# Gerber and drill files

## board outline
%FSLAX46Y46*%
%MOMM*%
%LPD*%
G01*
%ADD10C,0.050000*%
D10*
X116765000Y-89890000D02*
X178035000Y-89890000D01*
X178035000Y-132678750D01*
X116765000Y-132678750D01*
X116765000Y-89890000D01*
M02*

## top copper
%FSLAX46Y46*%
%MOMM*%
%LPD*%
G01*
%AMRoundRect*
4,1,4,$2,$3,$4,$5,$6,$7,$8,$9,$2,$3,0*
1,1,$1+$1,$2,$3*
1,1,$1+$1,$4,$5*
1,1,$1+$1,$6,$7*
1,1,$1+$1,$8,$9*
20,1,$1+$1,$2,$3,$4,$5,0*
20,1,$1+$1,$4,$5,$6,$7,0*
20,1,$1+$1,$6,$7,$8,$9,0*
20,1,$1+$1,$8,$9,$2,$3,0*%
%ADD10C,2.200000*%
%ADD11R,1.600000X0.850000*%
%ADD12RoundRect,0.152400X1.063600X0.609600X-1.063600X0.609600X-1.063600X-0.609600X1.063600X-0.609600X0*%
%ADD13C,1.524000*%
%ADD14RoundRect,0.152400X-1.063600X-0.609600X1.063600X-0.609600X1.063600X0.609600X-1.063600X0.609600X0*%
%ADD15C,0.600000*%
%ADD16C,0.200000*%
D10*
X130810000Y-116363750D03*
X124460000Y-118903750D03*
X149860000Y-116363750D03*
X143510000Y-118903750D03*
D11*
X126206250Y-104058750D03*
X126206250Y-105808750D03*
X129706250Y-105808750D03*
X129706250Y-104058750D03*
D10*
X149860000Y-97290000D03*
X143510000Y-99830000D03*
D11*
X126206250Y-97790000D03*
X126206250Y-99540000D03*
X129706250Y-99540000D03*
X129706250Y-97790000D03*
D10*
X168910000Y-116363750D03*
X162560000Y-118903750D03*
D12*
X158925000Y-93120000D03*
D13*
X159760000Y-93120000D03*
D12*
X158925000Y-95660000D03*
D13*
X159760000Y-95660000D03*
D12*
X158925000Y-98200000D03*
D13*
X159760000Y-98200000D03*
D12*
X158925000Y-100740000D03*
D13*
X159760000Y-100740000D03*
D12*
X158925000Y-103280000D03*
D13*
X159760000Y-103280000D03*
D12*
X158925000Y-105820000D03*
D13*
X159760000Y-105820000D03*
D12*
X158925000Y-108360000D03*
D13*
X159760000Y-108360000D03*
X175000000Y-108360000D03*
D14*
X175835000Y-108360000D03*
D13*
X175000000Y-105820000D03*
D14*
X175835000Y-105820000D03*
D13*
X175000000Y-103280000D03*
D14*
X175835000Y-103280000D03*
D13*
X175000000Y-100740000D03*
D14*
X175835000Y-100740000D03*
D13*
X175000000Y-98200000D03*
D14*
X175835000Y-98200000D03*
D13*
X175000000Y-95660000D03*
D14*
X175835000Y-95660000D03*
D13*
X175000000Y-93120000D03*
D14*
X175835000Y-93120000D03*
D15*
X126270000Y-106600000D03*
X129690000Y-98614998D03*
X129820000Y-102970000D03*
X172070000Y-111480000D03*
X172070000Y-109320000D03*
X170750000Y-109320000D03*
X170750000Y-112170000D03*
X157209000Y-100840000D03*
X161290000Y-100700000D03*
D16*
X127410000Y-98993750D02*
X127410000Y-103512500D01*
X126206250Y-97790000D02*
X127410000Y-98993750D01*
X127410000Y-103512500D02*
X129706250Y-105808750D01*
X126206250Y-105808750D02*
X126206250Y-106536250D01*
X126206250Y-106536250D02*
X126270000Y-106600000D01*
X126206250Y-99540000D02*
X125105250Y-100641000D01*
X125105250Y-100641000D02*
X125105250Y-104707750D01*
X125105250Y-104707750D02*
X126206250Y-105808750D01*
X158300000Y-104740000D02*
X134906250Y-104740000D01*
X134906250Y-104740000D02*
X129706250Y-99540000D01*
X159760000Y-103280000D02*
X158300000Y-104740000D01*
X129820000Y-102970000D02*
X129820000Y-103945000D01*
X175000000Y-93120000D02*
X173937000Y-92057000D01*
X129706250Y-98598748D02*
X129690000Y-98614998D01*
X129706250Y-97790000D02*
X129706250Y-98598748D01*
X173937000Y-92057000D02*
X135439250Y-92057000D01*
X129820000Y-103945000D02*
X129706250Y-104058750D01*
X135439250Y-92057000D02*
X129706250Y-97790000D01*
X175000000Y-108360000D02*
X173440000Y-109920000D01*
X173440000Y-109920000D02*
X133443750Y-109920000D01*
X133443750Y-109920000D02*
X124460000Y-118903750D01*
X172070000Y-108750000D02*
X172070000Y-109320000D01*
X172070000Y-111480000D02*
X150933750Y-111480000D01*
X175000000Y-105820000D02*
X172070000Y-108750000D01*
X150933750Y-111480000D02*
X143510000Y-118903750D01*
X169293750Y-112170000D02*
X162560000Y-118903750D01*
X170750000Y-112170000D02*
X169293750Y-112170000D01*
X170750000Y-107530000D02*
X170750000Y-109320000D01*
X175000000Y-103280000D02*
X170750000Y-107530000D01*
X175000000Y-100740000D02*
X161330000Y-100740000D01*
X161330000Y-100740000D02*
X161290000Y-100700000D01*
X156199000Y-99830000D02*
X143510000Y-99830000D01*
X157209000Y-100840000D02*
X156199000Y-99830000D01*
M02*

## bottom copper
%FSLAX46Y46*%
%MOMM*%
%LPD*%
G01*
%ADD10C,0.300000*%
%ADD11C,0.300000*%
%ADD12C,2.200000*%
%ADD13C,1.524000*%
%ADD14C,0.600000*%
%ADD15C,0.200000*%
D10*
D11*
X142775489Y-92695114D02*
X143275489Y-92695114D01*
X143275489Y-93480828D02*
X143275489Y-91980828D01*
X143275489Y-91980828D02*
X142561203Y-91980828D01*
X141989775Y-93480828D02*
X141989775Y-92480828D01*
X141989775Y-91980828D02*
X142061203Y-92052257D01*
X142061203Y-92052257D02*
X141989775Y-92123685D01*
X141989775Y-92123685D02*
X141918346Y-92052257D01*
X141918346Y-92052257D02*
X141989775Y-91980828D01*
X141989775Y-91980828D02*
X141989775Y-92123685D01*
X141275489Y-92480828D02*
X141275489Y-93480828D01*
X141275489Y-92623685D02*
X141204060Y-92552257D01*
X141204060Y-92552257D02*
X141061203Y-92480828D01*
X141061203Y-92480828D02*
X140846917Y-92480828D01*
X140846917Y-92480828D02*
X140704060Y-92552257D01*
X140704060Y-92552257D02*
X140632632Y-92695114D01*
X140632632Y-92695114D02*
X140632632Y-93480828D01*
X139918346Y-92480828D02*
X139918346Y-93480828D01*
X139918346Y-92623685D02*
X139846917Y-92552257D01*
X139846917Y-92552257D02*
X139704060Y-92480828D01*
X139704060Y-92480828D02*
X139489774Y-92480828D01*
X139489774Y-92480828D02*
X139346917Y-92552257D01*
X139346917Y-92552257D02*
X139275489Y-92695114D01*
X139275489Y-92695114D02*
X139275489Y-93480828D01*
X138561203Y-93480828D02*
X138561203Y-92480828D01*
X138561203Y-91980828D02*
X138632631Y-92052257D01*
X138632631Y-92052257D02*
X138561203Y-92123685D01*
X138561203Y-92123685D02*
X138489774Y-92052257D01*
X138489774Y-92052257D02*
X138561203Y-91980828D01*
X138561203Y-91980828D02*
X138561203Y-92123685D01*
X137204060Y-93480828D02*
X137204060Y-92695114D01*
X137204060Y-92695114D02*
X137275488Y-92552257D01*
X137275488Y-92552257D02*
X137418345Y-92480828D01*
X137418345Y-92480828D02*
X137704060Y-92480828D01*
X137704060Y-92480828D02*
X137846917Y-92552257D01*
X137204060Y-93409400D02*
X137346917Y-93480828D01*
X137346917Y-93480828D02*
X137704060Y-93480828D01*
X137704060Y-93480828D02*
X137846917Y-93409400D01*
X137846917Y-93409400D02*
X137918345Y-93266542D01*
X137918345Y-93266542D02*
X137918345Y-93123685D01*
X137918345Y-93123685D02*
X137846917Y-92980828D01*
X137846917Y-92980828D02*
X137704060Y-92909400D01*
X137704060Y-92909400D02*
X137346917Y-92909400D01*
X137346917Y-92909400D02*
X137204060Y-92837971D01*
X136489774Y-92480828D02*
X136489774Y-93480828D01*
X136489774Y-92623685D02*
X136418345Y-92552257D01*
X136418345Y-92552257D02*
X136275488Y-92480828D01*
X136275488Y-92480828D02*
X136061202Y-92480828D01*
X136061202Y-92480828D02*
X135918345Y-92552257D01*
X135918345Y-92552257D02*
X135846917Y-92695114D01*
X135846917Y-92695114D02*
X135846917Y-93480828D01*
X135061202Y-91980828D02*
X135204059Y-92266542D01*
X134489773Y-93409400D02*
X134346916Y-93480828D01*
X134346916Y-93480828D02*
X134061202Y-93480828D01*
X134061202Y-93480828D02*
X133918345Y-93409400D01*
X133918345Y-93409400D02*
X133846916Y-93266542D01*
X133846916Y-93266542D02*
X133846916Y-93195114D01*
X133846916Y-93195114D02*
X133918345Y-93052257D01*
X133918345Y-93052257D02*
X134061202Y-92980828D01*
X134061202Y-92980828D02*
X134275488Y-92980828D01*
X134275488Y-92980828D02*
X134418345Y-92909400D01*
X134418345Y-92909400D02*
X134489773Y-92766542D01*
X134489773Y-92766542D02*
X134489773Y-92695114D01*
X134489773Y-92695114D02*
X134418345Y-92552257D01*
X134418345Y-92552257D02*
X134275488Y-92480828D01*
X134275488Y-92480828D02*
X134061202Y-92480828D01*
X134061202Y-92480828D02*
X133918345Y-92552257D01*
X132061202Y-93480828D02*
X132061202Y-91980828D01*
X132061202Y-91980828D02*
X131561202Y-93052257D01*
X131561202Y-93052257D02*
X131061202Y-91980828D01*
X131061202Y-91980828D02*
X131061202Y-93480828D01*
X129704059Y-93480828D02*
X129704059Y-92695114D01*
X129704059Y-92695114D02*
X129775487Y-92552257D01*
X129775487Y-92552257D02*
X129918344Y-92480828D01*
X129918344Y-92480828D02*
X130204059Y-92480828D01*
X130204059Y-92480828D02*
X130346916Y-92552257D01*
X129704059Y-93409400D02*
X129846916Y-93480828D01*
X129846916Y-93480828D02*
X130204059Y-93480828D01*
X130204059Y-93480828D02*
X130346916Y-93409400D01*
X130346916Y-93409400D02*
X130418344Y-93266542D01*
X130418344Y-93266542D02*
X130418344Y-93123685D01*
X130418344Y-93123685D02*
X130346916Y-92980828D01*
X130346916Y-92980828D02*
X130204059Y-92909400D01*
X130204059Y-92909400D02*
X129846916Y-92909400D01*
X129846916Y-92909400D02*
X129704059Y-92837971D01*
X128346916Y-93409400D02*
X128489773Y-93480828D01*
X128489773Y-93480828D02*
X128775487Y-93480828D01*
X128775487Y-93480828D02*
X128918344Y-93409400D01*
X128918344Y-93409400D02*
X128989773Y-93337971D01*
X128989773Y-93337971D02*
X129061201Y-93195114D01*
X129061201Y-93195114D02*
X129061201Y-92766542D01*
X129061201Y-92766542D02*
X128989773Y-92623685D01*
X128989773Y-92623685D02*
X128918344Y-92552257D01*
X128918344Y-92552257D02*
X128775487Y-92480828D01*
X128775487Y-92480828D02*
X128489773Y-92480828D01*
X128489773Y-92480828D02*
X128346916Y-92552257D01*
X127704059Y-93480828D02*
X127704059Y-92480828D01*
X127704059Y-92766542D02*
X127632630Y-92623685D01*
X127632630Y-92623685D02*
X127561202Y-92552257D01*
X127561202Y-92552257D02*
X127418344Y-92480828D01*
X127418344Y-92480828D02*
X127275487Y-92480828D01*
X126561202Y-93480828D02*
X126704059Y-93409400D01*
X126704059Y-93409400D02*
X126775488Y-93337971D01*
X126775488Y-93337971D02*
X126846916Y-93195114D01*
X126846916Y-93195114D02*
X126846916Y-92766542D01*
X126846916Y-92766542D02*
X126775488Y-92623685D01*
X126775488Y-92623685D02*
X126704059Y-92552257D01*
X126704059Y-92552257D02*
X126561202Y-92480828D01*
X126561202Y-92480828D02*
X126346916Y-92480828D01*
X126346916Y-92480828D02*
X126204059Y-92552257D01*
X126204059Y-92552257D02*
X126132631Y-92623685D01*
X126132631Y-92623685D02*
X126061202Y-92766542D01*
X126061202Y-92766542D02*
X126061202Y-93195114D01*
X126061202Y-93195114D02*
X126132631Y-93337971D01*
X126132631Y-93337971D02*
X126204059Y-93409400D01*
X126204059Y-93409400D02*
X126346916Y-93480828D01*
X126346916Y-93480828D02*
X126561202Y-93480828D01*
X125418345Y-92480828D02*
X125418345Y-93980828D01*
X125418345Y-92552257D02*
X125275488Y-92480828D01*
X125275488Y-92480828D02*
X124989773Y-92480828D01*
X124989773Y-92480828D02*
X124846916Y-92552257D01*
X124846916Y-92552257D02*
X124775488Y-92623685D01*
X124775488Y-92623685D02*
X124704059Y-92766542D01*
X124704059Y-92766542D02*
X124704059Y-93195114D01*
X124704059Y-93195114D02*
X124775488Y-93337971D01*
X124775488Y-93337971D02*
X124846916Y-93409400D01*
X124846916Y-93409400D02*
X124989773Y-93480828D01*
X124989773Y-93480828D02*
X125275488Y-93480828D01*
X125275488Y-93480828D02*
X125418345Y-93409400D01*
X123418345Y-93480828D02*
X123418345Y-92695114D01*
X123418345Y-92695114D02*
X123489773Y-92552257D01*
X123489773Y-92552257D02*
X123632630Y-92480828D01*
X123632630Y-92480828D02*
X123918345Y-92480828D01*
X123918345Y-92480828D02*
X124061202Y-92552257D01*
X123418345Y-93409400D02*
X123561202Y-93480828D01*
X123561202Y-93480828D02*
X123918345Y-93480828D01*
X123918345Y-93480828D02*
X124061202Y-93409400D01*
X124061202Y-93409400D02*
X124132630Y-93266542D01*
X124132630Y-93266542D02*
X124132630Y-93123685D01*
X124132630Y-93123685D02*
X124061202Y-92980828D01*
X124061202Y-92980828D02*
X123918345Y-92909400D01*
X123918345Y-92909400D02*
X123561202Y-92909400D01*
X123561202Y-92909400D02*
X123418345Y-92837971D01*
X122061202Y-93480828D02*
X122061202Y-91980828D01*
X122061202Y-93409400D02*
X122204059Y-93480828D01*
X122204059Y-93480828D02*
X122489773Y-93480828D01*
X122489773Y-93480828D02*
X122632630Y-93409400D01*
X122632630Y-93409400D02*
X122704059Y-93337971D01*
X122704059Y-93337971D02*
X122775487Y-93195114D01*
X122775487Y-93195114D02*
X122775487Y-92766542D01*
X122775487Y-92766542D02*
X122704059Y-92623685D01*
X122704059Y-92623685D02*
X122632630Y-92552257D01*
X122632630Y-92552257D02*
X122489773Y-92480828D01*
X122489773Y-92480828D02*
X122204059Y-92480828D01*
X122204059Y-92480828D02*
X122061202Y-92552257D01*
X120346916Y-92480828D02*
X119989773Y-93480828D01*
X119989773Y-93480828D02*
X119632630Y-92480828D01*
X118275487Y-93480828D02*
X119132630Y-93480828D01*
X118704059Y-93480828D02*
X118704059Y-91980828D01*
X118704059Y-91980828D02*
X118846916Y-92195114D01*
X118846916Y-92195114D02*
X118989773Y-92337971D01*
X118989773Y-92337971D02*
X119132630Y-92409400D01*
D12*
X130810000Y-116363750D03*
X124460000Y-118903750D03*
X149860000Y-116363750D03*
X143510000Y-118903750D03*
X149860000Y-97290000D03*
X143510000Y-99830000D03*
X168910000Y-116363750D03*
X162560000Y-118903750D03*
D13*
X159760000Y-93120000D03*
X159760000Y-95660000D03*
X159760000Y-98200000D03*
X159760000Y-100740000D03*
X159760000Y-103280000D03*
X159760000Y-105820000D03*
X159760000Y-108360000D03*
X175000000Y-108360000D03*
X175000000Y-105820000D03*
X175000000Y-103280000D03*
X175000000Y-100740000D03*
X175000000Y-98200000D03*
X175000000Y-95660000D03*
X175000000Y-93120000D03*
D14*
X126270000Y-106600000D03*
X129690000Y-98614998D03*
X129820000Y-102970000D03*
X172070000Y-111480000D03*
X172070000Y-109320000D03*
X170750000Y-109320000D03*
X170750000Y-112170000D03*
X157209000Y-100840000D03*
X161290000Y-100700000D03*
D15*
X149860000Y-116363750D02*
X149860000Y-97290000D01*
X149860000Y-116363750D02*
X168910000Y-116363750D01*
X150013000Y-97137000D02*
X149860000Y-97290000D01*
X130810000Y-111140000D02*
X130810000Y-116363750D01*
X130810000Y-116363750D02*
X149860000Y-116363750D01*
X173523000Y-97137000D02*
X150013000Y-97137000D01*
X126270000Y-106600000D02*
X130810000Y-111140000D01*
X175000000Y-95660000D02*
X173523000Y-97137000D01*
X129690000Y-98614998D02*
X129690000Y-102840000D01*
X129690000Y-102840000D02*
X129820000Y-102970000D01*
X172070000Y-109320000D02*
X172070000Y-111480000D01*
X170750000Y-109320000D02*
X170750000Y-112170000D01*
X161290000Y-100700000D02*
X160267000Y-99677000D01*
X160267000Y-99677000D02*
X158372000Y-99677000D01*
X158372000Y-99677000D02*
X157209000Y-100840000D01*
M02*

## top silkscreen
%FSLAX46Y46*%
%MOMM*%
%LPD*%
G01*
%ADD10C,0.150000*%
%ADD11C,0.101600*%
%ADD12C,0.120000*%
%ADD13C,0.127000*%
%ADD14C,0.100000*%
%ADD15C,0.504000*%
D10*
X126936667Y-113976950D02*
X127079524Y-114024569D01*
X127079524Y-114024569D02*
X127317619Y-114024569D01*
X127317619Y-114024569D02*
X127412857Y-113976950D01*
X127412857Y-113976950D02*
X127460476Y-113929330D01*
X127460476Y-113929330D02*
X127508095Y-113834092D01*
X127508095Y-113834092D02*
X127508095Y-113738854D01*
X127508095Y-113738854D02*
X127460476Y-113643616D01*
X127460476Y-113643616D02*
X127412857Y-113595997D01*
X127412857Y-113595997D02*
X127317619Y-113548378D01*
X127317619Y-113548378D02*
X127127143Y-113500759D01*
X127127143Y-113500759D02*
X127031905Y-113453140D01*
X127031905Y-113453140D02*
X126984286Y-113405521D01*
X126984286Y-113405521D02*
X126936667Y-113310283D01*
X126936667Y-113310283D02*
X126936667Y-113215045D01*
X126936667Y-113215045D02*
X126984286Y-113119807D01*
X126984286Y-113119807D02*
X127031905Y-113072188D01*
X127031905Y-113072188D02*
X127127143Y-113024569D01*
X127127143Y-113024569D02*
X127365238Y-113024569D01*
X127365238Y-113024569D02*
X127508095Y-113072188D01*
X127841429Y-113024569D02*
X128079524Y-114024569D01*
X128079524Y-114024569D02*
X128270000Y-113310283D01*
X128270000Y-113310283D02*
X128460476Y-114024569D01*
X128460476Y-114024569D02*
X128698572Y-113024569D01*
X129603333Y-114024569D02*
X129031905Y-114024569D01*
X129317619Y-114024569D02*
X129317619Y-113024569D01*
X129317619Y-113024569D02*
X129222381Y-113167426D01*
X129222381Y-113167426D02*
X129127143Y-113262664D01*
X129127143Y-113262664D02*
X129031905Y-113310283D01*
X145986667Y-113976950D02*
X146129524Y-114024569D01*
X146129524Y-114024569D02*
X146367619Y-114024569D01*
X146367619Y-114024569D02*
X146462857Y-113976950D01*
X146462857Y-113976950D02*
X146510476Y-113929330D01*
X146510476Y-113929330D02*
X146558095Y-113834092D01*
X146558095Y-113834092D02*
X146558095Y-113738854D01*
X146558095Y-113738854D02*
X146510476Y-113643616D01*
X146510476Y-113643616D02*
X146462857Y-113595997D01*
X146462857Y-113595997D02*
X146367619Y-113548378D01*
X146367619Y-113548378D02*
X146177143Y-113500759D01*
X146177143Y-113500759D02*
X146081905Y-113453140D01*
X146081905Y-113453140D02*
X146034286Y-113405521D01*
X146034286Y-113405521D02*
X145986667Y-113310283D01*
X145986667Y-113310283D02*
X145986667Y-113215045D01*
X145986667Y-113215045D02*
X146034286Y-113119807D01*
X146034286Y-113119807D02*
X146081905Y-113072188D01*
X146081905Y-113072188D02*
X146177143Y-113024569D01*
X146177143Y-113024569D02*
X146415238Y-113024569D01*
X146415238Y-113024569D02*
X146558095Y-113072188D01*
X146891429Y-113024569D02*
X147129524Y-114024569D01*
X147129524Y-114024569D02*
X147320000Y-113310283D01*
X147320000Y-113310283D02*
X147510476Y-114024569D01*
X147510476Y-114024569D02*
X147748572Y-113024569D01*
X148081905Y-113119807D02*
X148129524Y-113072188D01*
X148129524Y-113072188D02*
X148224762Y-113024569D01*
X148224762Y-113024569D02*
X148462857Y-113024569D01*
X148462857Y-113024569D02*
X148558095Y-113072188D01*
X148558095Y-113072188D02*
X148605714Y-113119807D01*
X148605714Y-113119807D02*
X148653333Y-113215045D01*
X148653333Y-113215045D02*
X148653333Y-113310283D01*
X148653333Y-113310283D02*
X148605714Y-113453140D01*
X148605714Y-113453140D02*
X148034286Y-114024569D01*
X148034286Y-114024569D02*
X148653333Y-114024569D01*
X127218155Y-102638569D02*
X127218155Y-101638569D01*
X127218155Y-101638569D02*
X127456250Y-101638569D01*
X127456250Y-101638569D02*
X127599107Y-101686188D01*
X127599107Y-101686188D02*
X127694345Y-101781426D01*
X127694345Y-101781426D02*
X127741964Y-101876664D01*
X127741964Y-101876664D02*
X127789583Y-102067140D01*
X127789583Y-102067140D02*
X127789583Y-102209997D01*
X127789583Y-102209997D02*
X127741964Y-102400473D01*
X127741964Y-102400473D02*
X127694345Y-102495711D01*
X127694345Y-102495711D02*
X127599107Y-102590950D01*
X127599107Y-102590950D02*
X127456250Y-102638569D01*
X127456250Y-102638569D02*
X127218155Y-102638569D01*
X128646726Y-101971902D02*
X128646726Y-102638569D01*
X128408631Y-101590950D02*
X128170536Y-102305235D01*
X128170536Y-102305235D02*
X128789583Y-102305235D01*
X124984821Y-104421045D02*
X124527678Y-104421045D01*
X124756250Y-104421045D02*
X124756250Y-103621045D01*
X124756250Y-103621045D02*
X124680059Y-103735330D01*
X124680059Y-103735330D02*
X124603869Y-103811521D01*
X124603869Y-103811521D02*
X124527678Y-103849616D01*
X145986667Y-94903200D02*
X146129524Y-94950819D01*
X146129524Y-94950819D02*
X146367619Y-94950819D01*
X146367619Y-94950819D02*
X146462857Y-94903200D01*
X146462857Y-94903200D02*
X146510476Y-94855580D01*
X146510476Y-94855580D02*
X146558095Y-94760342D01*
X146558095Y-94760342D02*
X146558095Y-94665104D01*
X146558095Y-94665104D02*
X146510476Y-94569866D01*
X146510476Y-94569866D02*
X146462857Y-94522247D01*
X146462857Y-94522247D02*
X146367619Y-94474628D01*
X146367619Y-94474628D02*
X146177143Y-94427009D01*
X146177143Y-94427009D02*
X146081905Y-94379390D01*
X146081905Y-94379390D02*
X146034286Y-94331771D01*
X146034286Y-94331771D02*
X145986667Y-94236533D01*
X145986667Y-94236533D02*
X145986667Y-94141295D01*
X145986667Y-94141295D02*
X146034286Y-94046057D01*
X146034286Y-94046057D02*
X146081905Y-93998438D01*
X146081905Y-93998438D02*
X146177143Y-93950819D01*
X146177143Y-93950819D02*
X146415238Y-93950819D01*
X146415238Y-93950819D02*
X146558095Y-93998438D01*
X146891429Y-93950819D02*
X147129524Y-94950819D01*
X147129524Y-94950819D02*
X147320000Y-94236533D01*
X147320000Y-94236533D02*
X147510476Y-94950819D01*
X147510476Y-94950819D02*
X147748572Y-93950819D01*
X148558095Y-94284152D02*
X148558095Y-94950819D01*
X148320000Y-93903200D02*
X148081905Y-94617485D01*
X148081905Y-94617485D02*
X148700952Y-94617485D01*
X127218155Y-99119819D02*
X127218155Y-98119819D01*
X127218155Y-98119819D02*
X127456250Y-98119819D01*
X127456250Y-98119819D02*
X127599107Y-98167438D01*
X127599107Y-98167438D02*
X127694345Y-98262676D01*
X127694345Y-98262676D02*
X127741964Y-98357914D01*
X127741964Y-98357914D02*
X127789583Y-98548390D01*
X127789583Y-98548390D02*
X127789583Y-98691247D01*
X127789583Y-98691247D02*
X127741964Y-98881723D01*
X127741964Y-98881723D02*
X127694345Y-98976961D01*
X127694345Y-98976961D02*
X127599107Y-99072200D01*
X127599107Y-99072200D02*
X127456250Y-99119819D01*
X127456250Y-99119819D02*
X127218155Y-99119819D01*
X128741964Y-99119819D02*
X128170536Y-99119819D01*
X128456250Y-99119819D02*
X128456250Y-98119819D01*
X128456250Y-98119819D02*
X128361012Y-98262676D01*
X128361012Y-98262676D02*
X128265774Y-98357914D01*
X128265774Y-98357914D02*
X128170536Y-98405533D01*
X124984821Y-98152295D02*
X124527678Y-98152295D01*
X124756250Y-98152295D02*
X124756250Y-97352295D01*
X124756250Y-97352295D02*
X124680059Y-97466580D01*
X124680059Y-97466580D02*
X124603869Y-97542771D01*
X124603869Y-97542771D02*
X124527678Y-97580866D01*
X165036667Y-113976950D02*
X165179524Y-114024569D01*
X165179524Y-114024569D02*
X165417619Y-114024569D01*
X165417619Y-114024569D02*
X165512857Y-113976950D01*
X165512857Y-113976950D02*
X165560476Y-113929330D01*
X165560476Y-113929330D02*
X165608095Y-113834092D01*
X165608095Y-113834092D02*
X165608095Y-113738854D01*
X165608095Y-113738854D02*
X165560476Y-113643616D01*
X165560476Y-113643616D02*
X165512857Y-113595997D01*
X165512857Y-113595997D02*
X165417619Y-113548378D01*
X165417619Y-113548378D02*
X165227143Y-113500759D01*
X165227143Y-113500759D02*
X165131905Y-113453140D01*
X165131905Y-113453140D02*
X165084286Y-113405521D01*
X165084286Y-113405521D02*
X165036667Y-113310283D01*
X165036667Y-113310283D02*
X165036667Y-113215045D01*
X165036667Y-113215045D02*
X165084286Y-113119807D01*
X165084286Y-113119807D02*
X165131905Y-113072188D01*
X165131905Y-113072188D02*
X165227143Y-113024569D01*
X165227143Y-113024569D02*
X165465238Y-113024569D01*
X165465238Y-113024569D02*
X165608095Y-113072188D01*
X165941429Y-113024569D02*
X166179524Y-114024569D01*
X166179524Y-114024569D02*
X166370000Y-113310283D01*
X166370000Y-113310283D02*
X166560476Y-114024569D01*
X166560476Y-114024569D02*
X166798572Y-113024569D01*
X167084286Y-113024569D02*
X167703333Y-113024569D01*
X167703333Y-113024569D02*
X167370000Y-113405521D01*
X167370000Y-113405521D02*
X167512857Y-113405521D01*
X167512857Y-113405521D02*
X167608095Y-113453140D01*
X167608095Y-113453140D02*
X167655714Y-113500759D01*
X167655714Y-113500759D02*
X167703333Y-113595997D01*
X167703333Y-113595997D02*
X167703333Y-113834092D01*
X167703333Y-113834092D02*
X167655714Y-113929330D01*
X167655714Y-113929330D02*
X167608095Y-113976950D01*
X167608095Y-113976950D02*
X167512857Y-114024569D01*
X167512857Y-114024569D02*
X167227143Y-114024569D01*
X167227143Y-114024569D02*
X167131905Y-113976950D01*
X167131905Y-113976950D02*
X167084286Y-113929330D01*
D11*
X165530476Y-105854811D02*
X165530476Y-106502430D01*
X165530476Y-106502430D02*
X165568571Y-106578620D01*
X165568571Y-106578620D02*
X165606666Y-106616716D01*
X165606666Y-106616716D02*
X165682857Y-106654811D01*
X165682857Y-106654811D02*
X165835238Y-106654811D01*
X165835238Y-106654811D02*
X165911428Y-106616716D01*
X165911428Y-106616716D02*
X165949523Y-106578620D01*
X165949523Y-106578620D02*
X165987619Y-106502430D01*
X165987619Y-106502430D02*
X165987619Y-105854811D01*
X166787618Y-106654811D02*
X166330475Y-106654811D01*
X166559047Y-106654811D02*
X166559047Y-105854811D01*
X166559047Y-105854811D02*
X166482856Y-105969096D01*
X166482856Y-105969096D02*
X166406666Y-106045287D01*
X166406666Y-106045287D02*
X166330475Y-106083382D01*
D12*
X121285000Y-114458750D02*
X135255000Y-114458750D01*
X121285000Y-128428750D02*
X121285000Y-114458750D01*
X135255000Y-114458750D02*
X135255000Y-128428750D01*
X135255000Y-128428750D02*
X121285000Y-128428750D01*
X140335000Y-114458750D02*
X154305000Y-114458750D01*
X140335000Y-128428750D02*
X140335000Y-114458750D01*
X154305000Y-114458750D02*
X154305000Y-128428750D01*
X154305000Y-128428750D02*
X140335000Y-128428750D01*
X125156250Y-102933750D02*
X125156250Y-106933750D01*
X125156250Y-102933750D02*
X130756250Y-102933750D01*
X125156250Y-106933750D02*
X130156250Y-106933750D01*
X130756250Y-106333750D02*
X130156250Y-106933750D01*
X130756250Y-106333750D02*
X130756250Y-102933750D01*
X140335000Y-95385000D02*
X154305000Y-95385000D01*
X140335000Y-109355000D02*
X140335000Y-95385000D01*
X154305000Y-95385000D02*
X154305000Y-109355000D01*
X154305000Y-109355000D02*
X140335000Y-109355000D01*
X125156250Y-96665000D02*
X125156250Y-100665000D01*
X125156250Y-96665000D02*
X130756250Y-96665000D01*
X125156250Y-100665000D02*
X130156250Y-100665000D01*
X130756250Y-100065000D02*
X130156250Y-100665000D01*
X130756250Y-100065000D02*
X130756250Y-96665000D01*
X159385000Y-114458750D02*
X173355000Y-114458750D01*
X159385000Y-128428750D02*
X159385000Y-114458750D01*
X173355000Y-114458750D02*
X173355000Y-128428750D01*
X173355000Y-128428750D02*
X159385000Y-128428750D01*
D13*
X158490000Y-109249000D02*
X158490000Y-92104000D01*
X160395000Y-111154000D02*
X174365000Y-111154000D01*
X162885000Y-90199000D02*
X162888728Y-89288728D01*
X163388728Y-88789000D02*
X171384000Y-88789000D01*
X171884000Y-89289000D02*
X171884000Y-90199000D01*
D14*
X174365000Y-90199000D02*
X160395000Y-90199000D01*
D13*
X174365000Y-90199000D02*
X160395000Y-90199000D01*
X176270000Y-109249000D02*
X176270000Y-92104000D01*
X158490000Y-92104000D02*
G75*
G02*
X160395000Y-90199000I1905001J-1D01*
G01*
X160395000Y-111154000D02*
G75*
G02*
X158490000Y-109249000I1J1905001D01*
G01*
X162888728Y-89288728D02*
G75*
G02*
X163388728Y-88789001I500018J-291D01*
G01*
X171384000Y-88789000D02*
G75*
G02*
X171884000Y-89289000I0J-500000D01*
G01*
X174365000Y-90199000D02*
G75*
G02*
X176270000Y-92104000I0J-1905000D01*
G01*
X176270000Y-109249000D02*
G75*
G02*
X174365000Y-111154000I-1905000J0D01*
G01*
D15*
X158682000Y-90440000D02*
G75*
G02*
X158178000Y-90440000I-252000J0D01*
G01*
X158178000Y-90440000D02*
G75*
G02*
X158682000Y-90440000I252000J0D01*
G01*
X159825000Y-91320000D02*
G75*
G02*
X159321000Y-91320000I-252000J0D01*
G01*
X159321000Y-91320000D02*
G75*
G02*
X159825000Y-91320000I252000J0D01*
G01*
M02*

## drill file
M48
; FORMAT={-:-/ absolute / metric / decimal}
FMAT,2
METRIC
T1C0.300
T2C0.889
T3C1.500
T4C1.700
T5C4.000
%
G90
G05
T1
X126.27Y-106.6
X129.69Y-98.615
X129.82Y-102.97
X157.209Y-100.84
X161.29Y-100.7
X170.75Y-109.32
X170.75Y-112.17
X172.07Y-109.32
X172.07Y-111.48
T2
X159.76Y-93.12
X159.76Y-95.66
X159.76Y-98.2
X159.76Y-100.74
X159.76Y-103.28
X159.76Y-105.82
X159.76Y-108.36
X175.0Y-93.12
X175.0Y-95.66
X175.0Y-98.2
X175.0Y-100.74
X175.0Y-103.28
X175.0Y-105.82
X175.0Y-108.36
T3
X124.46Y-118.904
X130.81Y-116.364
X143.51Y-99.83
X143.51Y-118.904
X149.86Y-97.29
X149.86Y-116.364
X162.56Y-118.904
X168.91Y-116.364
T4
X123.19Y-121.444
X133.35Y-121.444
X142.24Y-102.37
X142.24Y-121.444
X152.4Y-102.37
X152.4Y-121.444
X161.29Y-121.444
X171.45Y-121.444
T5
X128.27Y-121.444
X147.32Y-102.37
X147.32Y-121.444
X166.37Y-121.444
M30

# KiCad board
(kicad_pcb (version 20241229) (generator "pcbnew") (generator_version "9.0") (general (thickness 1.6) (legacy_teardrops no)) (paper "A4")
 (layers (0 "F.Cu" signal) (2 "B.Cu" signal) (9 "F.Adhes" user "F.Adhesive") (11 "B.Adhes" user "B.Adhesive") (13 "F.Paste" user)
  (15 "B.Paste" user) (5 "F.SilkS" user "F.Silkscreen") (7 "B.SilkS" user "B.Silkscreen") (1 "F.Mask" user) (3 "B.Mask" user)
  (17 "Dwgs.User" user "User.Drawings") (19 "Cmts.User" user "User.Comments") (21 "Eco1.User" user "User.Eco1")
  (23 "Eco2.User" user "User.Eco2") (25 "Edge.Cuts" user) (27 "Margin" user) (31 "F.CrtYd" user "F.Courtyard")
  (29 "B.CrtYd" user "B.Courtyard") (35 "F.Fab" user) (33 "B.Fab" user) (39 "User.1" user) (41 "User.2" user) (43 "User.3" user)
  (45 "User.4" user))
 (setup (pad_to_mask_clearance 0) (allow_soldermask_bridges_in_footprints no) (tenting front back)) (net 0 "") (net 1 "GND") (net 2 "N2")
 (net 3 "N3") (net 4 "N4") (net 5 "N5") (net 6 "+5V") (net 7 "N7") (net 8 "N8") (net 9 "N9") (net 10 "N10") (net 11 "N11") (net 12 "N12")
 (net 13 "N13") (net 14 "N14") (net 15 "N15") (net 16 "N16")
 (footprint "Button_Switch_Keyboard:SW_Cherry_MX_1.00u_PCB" (layer "F.Cu") (at 130.81 116.36375)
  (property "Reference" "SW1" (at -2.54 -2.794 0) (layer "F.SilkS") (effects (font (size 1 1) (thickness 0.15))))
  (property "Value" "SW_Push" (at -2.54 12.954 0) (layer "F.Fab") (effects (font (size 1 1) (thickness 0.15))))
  (fp_line (start -9.525 -1.905) (end 4.445 -1.905) (stroke (width 0.12) (type solid)) (layer "F.SilkS"))
  (fp_line (start -9.525 12.065) (end -9.525 -1.905) (stroke (width 0.12) (type solid)) (layer "F.SilkS"))
  (fp_line (start 4.445 -1.905) (end 4.445 12.065) (stroke (width 0.12) (type solid)) (layer "F.SilkS"))
  (fp_line (start 4.445 12.065) (end -9.525 12.065) (stroke (width 0.12) (type solid)) (layer "F.SilkS"))
  (pad "" np_thru_hole circle (at -7.62 5.08) (size 1.7 1.7) (drill 1.7) (layers "*.Cu" "*.Mask"))
  (pad "" np_thru_hole circle (at -2.54 5.08) (size 4 4) (drill 4) (layers "*.Cu" "*.Mask"))
  (pad "" np_thru_hole circle (at 2.54 5.08) (size 1.7 1.7) (drill 1.7) (layers "*.Cu" "*.Mask"))
  (pad "1" thru_hole circle (at 0 0) (size 2.2 2.2) (drill 1.5) (layers "*.Cu" "*.Mask") (remove_unused_layers no) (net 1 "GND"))
  (pad "2" thru_hole circle (at -6.35 2.54) (size 2.2 2.2) (drill 1.5) (layers "*.Cu" "*.Mask") (remove_unused_layers no) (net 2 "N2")))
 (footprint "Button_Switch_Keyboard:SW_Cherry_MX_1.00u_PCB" (layer "F.Cu") (at 149.86 116.36375)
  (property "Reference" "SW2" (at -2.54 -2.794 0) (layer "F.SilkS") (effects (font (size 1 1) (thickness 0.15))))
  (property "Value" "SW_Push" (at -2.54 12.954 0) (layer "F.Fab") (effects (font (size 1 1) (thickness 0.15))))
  (fp_line (start -9.525 -1.905) (end 4.445 -1.905) (stroke (width 0.12) (type solid)) (layer "F.SilkS"))
  (fp_line (start -9.525 12.065) (end -9.525 -1.905) (stroke (width 0.12) (type solid)) (layer "F.SilkS"))
  (fp_line (start 4.445 -1.905) (end 4.445 12.065) (stroke (width 0.12) (type solid)) (layer "F.SilkS"))
  (fp_line (start 4.445 12.065) (end -9.525 12.065) (stroke (width 0.12) (type solid)) (layer "F.SilkS"))
  (pad "" np_thru_hole circle (at -7.62 5.08) (size 1.7 1.7) (drill 1.7) (layers "*.Cu" "*.Mask"))
  (pad "" np_thru_hole circle (at -2.54 5.08) (size 4 4) (drill 4) (layers "*.Cu" "*.Mask"))
  (pad "" np_thru_hole circle (at 2.54 5.08) (size 1.7 1.7) (drill 1.7) (layers "*.Cu" "*.Mask"))
  (pad "1" thru_hole circle (at 0 0) (size 2.2 2.2) (drill 1.5) (layers "*.Cu" "*.Mask") (remove_unused_layers no) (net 1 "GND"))
  (pad "2" thru_hole circle (at -6.35 2.54) (size 2.2 2.2) (drill 1.5) (layers "*.Cu" "*.Mask") (remove_unused_layers no) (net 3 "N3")))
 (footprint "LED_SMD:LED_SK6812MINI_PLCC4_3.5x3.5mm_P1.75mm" (layer "F.Cu") (at 127.95625 104.93375)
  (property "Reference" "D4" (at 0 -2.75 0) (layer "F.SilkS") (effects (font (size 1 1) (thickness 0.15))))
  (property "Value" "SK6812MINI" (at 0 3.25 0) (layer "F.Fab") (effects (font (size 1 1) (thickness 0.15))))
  (fp_line (start -2.8 -2) (end -2.8 2) (stroke (width 0.12) (type default)) (layer "F.SilkS"))
  (fp_line (start -2.8 -2) (end 2.8 -2) (stroke (width 0.12) (type solid)) (layer "F.SilkS"))
  (fp_line (start -2.8 2) (end 2.2 2) (stroke (width 0.12) (type solid)) (layer "F.SilkS"))
  (fp_line (start 2.8 1.4) (end 2.2 2) (stroke (width 0.12) (type default)) (layer "F.SilkS"))
  (fp_line (start 2.8 1.4) (end 2.8 -2) (stroke (width 0.12) (type solid)) (layer "F.SilkS"))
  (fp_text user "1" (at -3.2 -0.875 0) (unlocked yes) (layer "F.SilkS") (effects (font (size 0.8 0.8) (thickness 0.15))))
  (pad "1" smd rect (at -1.75 -0.875) (size 1.6 0.85) (layers "F.Cu" "F.Mask" "F.Paste") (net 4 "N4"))
  (pad "2" smd rect (at -1.75 0.875) (size 1.6 0.85) (layers "F.Cu" "F.Mask" "F.Paste") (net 1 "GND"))
  (pad "3" smd rect (at 1.75 0.875) (size 1.6 0.85) (layers "F.Cu" "F.Mask" "F.Paste") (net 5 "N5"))
  (pad "4" smd rect (at 1.75 -0.875) (size 1.6 0.85) (layers "F.Cu" "F.Mask" "F.Paste") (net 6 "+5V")))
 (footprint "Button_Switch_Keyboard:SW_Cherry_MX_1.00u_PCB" (layer "F.Cu") (at 149.86 97.29)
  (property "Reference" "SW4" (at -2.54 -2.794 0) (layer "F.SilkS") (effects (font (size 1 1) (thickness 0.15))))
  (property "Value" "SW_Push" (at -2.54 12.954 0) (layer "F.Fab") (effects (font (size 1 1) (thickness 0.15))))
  (fp_line (start -9.525 -1.905) (end 4.445 -1.905) (stroke (width 0.12) (type solid)) (layer "F.SilkS"))
  (fp_line (start -9.525 12.065) (end -9.525 -1.905) (stroke (width 0.12) (type solid)) (layer "F.SilkS"))
  (fp_line (start 4.445 -1.905) (end 4.445 12.065) (stroke (width 0.12) (type solid)) (layer "F.SilkS"))
  (fp_line (start 4.445 12.065) (end -9.525 12.065) (stroke (width 0.12) (type solid)) (layer "F.SilkS"))
  (pad "" np_thru_hole circle (at -7.62 5.08) (size 1.7 1.7) (drill 1.7) (layers "*.Cu" "*.Mask"))
  (pad "" np_thru_hole circle (at -2.54 5.08) (size 4 4) (drill 4) (layers "*.Cu" "*.Mask"))
  (pad "" np_thru_hole circle (at 2.54 5.08) (size 1.7 1.7) (drill 1.7) (layers "*.Cu" "*.Mask"))
  (pad "1" thru_hole circle (at 0 0) (size 2.2 2.2) (drill 1.5) (layers "*.Cu" "*.Mask") (remove_unused_layers no) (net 1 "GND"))
  (pad "2" thru_hole circle (at -6.35 2.54) (size 2.2 2.2) (drill 1.5) (layers "*.Cu" "*.Mask") (remove_unused_layers no) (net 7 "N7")))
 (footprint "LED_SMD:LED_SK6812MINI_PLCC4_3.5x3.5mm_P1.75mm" (layer "F.Cu") (at 127.95625 98.665)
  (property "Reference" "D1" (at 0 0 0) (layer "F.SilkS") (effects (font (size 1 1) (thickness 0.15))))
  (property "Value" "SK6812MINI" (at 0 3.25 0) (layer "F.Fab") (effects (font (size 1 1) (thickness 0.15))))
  (fp_line (start -2.8 -2) (end -2.8 2) (stroke (width 0.12) (type default)) (layer "F.SilkS"))
  (fp_line (start -2.8 -2) (end 2.8 -2) (stroke (width 0.12) (type solid)) (layer "F.SilkS"))
  (fp_line (start -2.8 2) (end 2.2 2) (stroke (width 0.12) (type solid)) (layer "F.SilkS"))
  (fp_line (start 2.8 1.4) (end 2.2 2) (stroke (width 0.12) (type default)) (layer "F.SilkS"))
  (fp_line (start 2.8 1.4) (end 2.8 -2) (stroke (width 0.12) (type solid)) (layer "F.SilkS"))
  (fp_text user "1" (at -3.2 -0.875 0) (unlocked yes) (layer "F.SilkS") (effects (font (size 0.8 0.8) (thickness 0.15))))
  (pad "1" smd rect (at -1.75 -0.875) (size 1.6 0.85) (layers "F.Cu" "F.Mask" "F.Paste") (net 5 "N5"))
  (pad "2" smd rect (at -1.75 0.875) (size 1.6 0.85) (layers "F.Cu" "F.Mask" "F.Paste") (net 1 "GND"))
  (pad "3" smd rect (at 1.75 0.875) (size 1.6 0.85) (layers "F.Cu" "F.Mask" "F.Paste") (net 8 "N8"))
  (pad "4" smd rect (at 1.75 -0.875) (size 1.6 0.85) (layers "F.Cu" "F.Mask" "F.Paste") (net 6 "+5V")))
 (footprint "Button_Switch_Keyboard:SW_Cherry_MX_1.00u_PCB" (layer "F.Cu") (at 168.91 116.36375)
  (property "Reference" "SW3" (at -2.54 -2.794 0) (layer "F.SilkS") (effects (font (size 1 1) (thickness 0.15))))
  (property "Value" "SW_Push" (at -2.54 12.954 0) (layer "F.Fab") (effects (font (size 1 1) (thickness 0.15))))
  (fp_line (start -9.525 -1.905) (end 4.445 -1.905) (stroke (width 0.12) (type solid)) (layer "F.SilkS"))
  (fp_line (start -9.525 12.065) (end -9.525 -1.905) (stroke (width 0.12) (type solid)) (layer "F.SilkS"))
  (fp_line (start 4.445 -1.905) (end 4.445 12.065) (stroke (width 0.12) (type solid)) (layer "F.SilkS"))
  (fp_line (start 4.445 12.065) (end -9.525 12.065) (stroke (width 0.12) (type solid)) (layer "F.SilkS"))
  (pad "" np_thru_hole circle (at -7.62 5.08) (size 1.7 1.7) (drill 1.7) (layers "*.Cu" "*.Mask"))
  (pad "" np_thru_hole circle (at -2.54 5.08) (size 4 4) (drill 4) (layers "*.Cu" "*.Mask"))
  (pad "" np_thru_hole circle (at 2.54 5.08) (size 1.7 1.7) (drill 1.7) (layers "*.Cu" "*.Mask"))
  (pad "1" thru_hole circle (at 0 0) (size 2.2 2.2) (drill 1.5) (layers "*.Cu" "*.Mask") (remove_unused_layers no) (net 1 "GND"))
  (pad "2" thru_hole circle (at -6.35 2.54) (size 2.2 2.2) (drill 1.5) (layers "*.Cu" "*.Mask") (remove_unused_layers no) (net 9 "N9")))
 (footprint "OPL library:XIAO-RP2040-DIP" (layer "F.Cu") (at 167.38 100.74)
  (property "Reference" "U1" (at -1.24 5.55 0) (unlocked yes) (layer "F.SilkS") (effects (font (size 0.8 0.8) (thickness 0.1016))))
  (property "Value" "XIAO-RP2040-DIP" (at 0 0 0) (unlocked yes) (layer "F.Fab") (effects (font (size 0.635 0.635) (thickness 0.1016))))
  (fp_line (start -8.89 8.509) (end -8.89 -8.636) (stroke (width 0.127) (type solid)) (layer "F.SilkS"))
  (fp_line (start -6.985 10.414) (end 6.985 10.414) (stroke (width 0.127) (type solid)) (layer "F.SilkS"))
  (fp_line (start -4.495 -10.541) (end -4.491272 -11.451272) (stroke (width 0.127) (type solid)) (layer "F.SilkS"))
  (fp_line (start -3.991272 -11.951) (end 4.004 -11.951) (stroke (width 0.127) (type solid)) (layer "F.SilkS"))
  (fp_line (start 4.504 -11.451) (end 4.504 -10.541) (stroke (width 0.127) (type solid)) (layer "F.SilkS"))
  (fp_line (start 6.985 -10.541) (end -6.985 -10.541) (stroke (width 0.1) (type solid)) (layer "F.SilkS"))
  (fp_line (start 6.985 -10.541) (end -6.985 -10.541) (stroke (width 0.127) (type solid)) (layer "F.SilkS"))
  (fp_line (start 8.89 8.509) (end 8.89 -8.636) (stroke (width 0.127) (type solid)) (layer "F.SilkS"))
  (fp_arc (start -8.89 -8.636) (mid -8.332038 -9.983038) (end -6.985 -10.541) (stroke (width 0.127) (type solid)) (layer "F.SilkS"))
  (fp_arc (start -6.985 10.414) (mid -8.332038 9.856038) (end -8.89 8.509) (stroke (width 0.127) (type solid)) (layer "F.SilkS"))
  (fp_arc (start -4.491272 -11.451272) (mid -4.344728 -11.80464) (end -3.991272 -11.951) (stroke (width 0.127) (type default))
   (layer "F.SilkS"))
  (fp_arc (start 4.004 -11.951) (mid 4.357553 -11.804553) (end 4.504 -11.451) (stroke (width 0.127) (type default)) (layer "F.SilkS"))
  (fp_arc (start 6.985 -10.541) (mid 8.332038 -9.983038) (end 8.89 -8.636) (stroke (width 0.127) (type solid)) (layer "F.SilkS"))
  (fp_arc (start 8.89 8.509) (mid 8.332038 9.856038) (end 6.985 10.414) (stroke (width 0.127) (type solid)) (layer "F.SilkS"))
  (fp_circle (center -8.95 -10.3) (end -8.95 -10.554) (stroke (width 0.5) (type solid)) (fill yes) (layer "F.SilkS"))
  (fp_circle (center -7.807 -9.42) (end -7.807 -9.674) (stroke (width 0.5) (type solid)) (fill yes) (layer "F.SilkS"))
  (pad "1" smd roundrect (at -8.455 -7.62 180) (size 2.432 1.524) (layers "F.Cu" "F.Mask") (roundrect_rratio 0.1) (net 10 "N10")
   (thermal_bridge_angle 45))
  (pad "1" thru_hole circle (at -7.62 -7.62 180) (size 1.524 1.524) (drill 0.889) (layers "*.Cu" "*.Mask") (remove_unused_layers no)
   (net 10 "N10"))
  (pad "2" smd roundrect (at -8.455 -5.08 180) (size 2.432 1.524) (layers "F.Cu" "F.Mask") (roundrect_rratio 0.1) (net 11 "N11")
   (thermal_bridge_angle 45))
  (pad "2" thru_hole circle (at -7.62 -5.08 180) (size 1.524 1.524) (drill 0.889) (layers "*.Cu" "*.Mask") (remove_unused_layers no)
   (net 11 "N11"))
  (pad "3" smd roundrect (at -8.455 -2.54 180) (size 2.432 1.524) (layers "F.Cu" "F.Mask") (roundrect_rratio 0.1) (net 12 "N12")
   (thermal_bridge_angle 45))
  (pad "3" thru_hole circle (at -7.62 -2.54 180) (size 1.524 1.524) (drill 0.889) (layers "*.Cu" "*.Mask") (remove_unused_layers no)
   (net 12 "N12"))
  (pad "4" smd roundrect (at -8.455 0 180) (size 2.432 1.524) (layers "F.Cu" "F.Mask") (roundrect_rratio 0.1) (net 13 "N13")
   (thermal_bridge_angle 45))
  (pad "4" thru_hole circle (at -7.62 0 180) (size 1.524 1.524) (drill 0.889) (layers "*.Cu" "*.Mask") (remove_unused_layers no)
   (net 13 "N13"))
  (pad "5" smd roundrect (at -8.455 2.54 180) (size 2.432 1.524) (layers "F.Cu" "F.Mask") (roundrect_rratio 0.1) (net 8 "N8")
   (thermal_bridge_angle 45))
  (pad "5" thru_hole circle (at -7.62 2.54 180) (size 1.524 1.524) (drill 0.889) (layers "*.Cu" "*.Mask") (remove_unused_layers no)
   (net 8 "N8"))
  (pad "6" smd roundrect (at -8.455 5.08 180) (size 2.432 1.524) (layers "F.Cu" "F.Mask") (roundrect_rratio 0.1) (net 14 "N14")
   (thermal_bridge_angle 45))
  (pad "6" thru_hole circle (at -7.62 5.08 180) (size 1.524 1.524) (drill 0.889) (layers "*.Cu" "*.Mask") (remove_unused_layers no)
   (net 14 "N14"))
  (pad "7" smd roundrect (at -8.455 7.62 180) (size 2.432 1.524) (layers "F.Cu" "F.Mask") (roundrect_rratio 0.1) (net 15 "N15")
   (thermal_bridge_angle 45))
  (pad "7" thru_hole circle (at -7.62 7.62 180) (size 1.524 1.524) (drill 0.889) (layers "*.Cu" "*.Mask") (remove_unused_layers no)
   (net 15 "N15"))
  (pad "8" thru_hole circle (at 7.62 7.62) (size 1.524 1.524) (drill 0.889) (layers "*.Cu" "*.Mask") (remove_unused_layers no) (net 2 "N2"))
  (pad "8" smd roundrect (at 8.455 7.62) (size 2.432 1.524) (layers "F.Cu" "F.Mask") (roundrect_rratio 0.1) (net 2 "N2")
   (thermal_bridge_angle 45))
  (pad "9" thru_hole circle (at 7.62 5.08) (size 1.524 1.524) (drill 0.889) (layers "*.Cu" "*.Mask") (remove_unused_layers no) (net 3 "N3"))
  (pad "9" smd roundrect (at 8.455 5.08) (size 2.432 1.524) (layers "F.Cu" "F.Mask") (roundrect_rratio 0.1) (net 3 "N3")
   (thermal_bridge_angle 45))
  (pad "10" thru_hole circle (at 7.62 2.54) (size 1.524 1.524) (drill 0.889) (layers "*.Cu" "*.Mask") (remove_unused_layers no) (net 9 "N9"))
  (pad "10" smd roundrect (at 8.455 2.54) (size 2.432 1.524) (layers "F.Cu" "F.Mask") (roundrect_rratio 0.1) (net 9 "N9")
   (thermal_bridge_angle 45))
  (pad "11" thru_hole circle (at 7.62 0) (size 1.524 1.524) (drill 0.889) (layers "*.Cu" "*.Mask") (remove_unused_layers no) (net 7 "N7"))
  (pad "11" smd roundrect (at 8.455 0) (size 2.432 1.524) (layers "F.Cu" "F.Mask") (roundrect_rratio 0.1) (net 7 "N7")
   (thermal_bridge_angle 45))
  (pad "12" thru_hole circle (at 7.62 -2.54) (size 1.524 1.524) (drill 0.889) (layers "*.Cu" "*.Mask") (remove_unused_layers no)
   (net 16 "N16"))
  (pad "12" smd roundrect (at 8.455 -2.54) (size 2.432 1.524) (layers "F.Cu" "F.Mask") (roundrect_rratio 0.1) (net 16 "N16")
   (thermal_bridge_angle 45))
  (pad "13" thru_hole circle (at 7.62 -5.08) (size 1.524 1.524) (drill 0.889) (layers "*.Cu" "*.Mask") (remove_unused_layers no)
   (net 1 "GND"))
  (pad "13" smd roundrect (at 8.455 -5.08) (size 2.432 1.524) (layers "F.Cu" "F.Mask") (roundrect_rratio 0.1) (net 1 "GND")
   (thermal_bridge_angle 45))
  (pad "14" thru_hole circle (at 7.62 -7.62) (size 1.524 1.524) (drill 0.889) (layers "*.Cu" "*.Mask") (remove_unused_layers no)
   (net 6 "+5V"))
  (pad "14" smd roundrect (at 8.455 -7.62) (size 2.432 1.524) (layers "F.Cu" "F.Mask") (roundrect_rratio 0.1) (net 6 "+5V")
   (thermal_bridge_angle 45)))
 (gr_rect (start 116.765 89.89) (end 178.035 132.67875) (stroke (width 0.05) (type default)) (fill no) (layer "Edge.Cuts"))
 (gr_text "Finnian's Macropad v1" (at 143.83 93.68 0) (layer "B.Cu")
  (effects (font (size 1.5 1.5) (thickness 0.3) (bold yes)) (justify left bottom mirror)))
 (segment (start 127.41 98.99375) (end 127.41 103.5125) (width 0.2) (layer "F.Cu") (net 5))
 (segment (start 126.20625 97.79) (end 127.41 98.99375) (width 0.2) (layer "F.Cu") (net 5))
 (segment (start 127.41 103.5125) (end 129.70625 105.80875) (width 0.2) (layer "F.Cu") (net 5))
 (segment (start 126.20625 105.80875) (end 126.20625 106.53625) (width 0.2) (layer "F.Cu") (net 1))
 (segment (start 126.20625 106.53625) (end 126.27 106.6) (width 0.2) (layer "F.Cu") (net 1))
 (segment (start 126.20625 99.54) (end 125.10525 100.641) (width 0.2) (layer "F.Cu") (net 1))
 (segment (start 125.10525 100.641) (end 125.10525 104.70775) (width 0.2) (layer "F.Cu") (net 1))
 (segment (start 125.10525 104.70775) (end 126.20625 105.80875) (width 0.2) (layer "F.Cu") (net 1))
 (via (at 126.27 106.6) (size 0.6) (drill 0.3) (layers "F.Cu" "B.Cu") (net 1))
 (segment (start 149.86 116.36375) (end 149.86 97.29) (width 0.2) (layer "B.Cu") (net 1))
 (segment (start 149.86 116.36375) (end 168.91 116.36375) (width 0.2) (layer "B.Cu") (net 1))
 (segment (start 150.013 97.137) (end 149.86 97.29) (width 0.2) (layer "B.Cu") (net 1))
 (segment (start 130.81 111.14) (end 130.81 116.36375) (width 0.2) (layer "B.Cu") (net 1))
 (segment (start 130.81 116.36375) (end 149.86 116.36375) (width 0.2) (layer "B.Cu") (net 1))
 (segment (start 173.523 97.137) (end 150.013 97.137) (width 0.2) (layer "B.Cu") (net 1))
 (segment (start 126.27 106.6) (end 130.81 111.14) (width 0.2) (layer "B.Cu") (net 1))
 (segment (start 175 95.66) (end 173.523 97.137) (width 0.2) (layer "B.Cu") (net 1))
 (segment (start 158.3 104.74) (end 134.90625 104.74) (width 0.2) (layer "F.Cu") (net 8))
 (segment (start 134.90625 104.74) (end 129.70625 99.54) (width 0.2) (layer "F.Cu") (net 8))
 (segment (start 159.76 103.28) (end 158.3 104.74) (width 0.2) (layer "F.Cu") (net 8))
 (segment (start 129.82 102.97) (end 129.82 103.945) (width 0.2) (layer "F.Cu") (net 6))
 (segment (start 175 93.12) (end 173.937 92.057) (width 0.2) (layer "F.Cu") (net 6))
 (segment (start 129.70625 98.598748) (end 129.69 98.614998) (width 0.2) (layer "F.Cu") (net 6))
 (segment (start 129.70625 97.79) (end 129.70625 98.598748) (width 0.2) (layer "F.Cu") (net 6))
 (segment (start 173.937 92.057) (end 135.43925 92.057) (width 0.2) (layer "F.Cu") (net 6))
 (segment (start 129.82 103.945) (end 129.70625 104.05875) (width 0.2) (layer "F.Cu") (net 6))
 (segment (start 135.43925 92.057) (end 129.70625 97.79) (width 0.2) (layer "F.Cu") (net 6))
 (via (at 129.69 98.614998) (size 0.6) (drill 0.3) (layers "F.Cu" "B.Cu") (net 6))
 (via (at 129.82 102.97) (size 0.6) (drill 0.3) (layers "F.Cu" "B.Cu") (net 6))
 (segment (start 129.69 98.614998) (end 129.69 102.84) (width 0.2) (layer "B.Cu") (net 6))
 (segment (start 129.69 102.84) (end 129.82 102.97) (width 0.2) (layer "B.Cu") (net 6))
 (segment (start 175 108.36) (end 173.44 109.92) (width 0.2) (layer "F.Cu") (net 2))
 (segment (start 173.44 109.92) (end 133.44375 109.92) (width 0.2) (layer "F.Cu") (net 2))
 (segment (start 133.44375 109.92) (end 124.46 118.90375) (width 0.2) (layer "F.Cu") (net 2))
 (segment (start 172.07 108.75) (end 172.07 109.32) (width 0.2) (layer "F.Cu") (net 3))
 (segment (start 172.07 111.48) (end 150.93375 111.48) (width 0.2) (layer "F.Cu") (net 3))
 (segment (start 175 105.82) (end 172.07 108.75) (width 0.2) (layer "F.Cu") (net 3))
 (segment (start 150.93375 111.48) (end 143.51 118.90375) (width 0.2) (layer "F.Cu") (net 3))
 (via (at 172.07 111.48) (size 0.6) (drill 0.3) (layers "F.Cu" "B.Cu") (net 3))
 (via (at 172.07 109.32) (size 0.6) (drill 0.3) (layers "F.Cu" "B.Cu") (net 3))
 (segment (start 172.07 109.32) (end 172.07 111.48) (width 0.2) (layer "B.Cu") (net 3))
 (segment (start 169.29375 112.17) (end 162.56 118.90375) (width 0.2) (layer "F.Cu") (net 9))
 (segment (start 170.75 112.17) (end 169.29375 112.17) (width 0.2) (layer "F.Cu") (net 9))
 (segment (start 170.75 107.53) (end 170.75 109.32) (width 0.2) (layer "F.Cu") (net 9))
 (segment (start 175 103.28) (end 170.75 107.53) (width 0.2) (layer "F.Cu") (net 9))
 (via (at 170.75 109.32) (size 0.6) (drill 0.3) (layers "F.Cu" "B.Cu") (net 9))
 (via (at 170.75 112.17) (size 0.6) (drill 0.3) (layers "F.Cu" "B.Cu") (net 9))
 (segment (start 170.75 109.32) (end 170.75 112.17) (width 0.2) (layer "B.Cu") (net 9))
 (segment (start 175 100.74) (end 161.33 100.74) (width 0.2) (layer "F.Cu") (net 7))
 (segment (start 161.33 100.74) (end 161.29 100.7) (width 0.2) (layer "F.Cu") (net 7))
 (segment (start 156.199 99.83) (end 143.51 99.83) (width 0.2) (layer "F.Cu") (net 7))
 (segment (start 157.209 100.84) (end 156.199 99.83) (width 0.2) (layer "F.Cu") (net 7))
 (via (at 157.209 100.84) (size 0.6) (drill 0.3) (layers "F.Cu" "B.Cu") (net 7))
 (via (at 161.29 100.7) (size 0.6) (drill 0.3) (layers "F.Cu" "B.Cu") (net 7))
 (segment (start 161.29 100.7) (end 160.267 99.677) (width 0.2) (layer "B.Cu") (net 7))
 (segment (start 160.267 99.677) (end 158.372 99.677) (width 0.2) (layer "B.Cu") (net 7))
 (segment (start 158.372 99.677) (end 157.209 100.84) (width 0.2) (layer "B.Cu") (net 7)))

